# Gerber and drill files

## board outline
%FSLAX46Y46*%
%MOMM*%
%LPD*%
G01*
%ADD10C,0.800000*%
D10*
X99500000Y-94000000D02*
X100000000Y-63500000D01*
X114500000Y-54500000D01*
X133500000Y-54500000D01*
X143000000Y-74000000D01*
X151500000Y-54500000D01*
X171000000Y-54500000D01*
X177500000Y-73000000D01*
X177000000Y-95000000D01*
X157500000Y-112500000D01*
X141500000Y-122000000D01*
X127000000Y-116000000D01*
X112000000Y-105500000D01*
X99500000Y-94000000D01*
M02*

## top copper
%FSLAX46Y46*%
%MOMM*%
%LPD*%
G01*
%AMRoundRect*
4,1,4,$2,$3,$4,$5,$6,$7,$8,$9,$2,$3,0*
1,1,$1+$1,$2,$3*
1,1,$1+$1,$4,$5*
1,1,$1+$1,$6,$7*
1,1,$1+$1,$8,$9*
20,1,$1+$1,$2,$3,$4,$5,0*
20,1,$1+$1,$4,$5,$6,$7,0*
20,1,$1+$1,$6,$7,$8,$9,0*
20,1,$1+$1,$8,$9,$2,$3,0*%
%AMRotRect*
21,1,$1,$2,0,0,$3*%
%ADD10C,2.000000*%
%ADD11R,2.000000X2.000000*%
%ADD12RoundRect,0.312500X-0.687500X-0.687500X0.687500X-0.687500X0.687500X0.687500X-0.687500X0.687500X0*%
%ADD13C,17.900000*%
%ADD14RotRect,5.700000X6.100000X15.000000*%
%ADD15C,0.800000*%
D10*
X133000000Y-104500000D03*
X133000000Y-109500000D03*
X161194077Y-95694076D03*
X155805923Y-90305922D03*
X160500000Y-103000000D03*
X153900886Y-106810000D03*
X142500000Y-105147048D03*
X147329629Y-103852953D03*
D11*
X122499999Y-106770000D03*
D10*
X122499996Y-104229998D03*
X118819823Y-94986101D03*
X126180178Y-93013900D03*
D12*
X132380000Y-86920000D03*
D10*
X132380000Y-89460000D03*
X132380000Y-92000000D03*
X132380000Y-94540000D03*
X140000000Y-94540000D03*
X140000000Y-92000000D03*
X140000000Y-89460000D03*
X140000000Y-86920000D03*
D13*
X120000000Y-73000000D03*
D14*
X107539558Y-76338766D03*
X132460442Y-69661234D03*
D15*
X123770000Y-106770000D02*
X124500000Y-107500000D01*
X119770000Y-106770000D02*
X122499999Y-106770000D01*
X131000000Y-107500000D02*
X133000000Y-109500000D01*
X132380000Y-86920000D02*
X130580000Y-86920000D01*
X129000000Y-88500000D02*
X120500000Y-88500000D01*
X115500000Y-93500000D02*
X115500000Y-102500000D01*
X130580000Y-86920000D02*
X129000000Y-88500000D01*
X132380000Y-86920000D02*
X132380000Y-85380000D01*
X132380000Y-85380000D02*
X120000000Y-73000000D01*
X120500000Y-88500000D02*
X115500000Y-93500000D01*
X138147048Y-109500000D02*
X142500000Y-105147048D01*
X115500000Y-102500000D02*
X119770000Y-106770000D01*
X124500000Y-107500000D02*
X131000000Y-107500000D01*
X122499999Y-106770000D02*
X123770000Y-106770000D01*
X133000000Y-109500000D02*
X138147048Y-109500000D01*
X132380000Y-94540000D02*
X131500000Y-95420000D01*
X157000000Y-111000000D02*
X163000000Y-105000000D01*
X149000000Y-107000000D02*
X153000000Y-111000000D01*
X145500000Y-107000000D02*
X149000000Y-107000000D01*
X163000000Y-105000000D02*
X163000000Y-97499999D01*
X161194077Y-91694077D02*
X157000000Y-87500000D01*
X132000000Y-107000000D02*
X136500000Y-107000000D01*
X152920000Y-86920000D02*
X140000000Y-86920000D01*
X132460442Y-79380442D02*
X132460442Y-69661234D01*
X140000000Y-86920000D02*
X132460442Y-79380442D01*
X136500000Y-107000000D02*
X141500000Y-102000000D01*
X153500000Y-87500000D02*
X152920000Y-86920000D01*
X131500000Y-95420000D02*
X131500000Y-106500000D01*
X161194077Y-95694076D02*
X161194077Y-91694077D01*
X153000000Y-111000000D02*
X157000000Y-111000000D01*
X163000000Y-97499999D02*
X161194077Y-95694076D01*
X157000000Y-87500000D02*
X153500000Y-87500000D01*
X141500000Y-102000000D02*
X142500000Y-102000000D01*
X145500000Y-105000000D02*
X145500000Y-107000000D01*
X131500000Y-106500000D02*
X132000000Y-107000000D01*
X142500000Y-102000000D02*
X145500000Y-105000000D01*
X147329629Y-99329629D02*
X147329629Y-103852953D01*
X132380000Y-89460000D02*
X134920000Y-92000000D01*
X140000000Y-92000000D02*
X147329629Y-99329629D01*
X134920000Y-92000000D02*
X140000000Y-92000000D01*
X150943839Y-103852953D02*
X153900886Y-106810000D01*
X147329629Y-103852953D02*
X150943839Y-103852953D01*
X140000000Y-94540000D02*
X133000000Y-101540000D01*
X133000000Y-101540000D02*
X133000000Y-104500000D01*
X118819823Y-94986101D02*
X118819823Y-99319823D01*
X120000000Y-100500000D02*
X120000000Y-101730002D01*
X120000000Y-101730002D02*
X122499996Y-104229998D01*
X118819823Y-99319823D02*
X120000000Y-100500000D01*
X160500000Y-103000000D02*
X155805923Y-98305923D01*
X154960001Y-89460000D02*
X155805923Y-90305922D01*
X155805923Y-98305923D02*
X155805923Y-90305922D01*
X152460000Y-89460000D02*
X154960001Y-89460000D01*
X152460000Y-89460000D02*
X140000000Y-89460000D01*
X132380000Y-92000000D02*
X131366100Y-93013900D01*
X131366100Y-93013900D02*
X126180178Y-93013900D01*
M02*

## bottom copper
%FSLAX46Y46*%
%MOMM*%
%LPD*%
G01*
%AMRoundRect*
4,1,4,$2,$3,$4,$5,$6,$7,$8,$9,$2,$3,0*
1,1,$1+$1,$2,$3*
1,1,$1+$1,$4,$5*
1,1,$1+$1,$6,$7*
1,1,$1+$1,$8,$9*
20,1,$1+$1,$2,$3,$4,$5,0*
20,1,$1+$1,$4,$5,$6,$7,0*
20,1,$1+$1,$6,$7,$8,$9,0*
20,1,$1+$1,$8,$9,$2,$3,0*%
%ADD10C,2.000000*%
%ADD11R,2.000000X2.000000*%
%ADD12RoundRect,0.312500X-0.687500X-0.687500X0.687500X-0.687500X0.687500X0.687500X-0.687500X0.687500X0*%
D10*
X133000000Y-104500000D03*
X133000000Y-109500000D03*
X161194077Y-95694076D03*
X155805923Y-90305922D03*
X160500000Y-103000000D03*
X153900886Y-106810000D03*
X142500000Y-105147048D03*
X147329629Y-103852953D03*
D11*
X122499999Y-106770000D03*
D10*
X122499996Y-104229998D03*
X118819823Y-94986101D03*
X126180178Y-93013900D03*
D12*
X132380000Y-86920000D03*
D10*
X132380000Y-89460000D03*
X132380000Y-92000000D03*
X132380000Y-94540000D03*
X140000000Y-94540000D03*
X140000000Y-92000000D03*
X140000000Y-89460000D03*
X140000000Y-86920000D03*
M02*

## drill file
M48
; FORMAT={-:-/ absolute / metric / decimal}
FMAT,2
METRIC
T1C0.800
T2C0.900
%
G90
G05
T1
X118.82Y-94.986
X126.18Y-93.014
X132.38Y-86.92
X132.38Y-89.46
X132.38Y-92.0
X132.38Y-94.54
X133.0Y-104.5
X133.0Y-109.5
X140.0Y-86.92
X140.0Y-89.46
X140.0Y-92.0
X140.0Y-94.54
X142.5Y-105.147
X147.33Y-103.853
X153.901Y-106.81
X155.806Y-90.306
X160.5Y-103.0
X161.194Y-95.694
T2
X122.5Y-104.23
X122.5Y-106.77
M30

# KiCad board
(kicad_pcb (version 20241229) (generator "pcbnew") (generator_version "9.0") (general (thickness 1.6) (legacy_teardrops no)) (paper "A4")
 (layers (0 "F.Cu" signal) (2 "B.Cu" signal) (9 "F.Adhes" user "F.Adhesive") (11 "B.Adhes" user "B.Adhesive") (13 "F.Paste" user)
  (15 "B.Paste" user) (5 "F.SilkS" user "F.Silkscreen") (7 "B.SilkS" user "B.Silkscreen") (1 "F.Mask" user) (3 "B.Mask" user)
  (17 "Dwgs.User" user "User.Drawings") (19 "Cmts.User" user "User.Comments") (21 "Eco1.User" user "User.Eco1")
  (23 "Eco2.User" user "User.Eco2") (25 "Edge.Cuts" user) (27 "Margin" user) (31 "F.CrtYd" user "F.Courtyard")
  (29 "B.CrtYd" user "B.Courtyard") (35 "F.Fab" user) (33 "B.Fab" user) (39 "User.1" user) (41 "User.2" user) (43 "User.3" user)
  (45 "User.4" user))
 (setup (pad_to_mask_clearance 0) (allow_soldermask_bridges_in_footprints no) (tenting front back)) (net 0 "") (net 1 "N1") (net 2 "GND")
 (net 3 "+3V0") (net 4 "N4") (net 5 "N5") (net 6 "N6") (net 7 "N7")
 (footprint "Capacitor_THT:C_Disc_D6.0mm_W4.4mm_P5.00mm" (layer "F.Cu") (at 133 104.5 -90)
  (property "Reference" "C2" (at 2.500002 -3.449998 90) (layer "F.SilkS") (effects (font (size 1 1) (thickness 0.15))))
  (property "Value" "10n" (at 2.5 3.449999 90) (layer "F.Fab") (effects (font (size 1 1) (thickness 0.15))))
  (pad "1" thru_hole circle (at 0 0 270) (size 2 2) (drill 0.8) (layers "*.Cu" "*.Mask") (remove_unused_layers no) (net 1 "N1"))
  (pad "2" thru_hole circle (at 5 0 270) (size 2 2) (drill 0.8) (layers "*.Cu" "*.Mask") (remove_unused_layers no) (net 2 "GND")))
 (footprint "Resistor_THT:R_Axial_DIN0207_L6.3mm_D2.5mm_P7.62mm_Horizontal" (layer "F.Cu") (at 161.194077 95.694076 135)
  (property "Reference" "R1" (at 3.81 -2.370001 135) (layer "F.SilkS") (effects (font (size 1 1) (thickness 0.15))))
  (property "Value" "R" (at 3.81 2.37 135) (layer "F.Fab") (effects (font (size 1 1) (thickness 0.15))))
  (pad "1" thru_hole circle (at 0 0 135) (size 2 2) (drill 0.8) (layers "*.Cu" "*.Mask") (remove_unused_layers no) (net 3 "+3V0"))
  (pad "2" thru_hole circle (at 7.62 0 135) (size 2 2) (drill 0.8) (layers "*.Cu" "*.Mask") (remove_unused_layers no) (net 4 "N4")))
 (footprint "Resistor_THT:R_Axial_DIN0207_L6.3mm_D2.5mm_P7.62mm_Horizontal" (layer "F.Cu") (at 160.5 103 -150)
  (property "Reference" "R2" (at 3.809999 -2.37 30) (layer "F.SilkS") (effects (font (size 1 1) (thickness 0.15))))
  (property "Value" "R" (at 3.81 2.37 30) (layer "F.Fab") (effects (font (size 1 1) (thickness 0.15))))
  (pad "1" thru_hole circle (at 0 0 210) (size 2 2) (drill 0.8) (layers "*.Cu" "*.Mask") (remove_unused_layers no) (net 4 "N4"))
  (pad "2" thru_hole circle (at 7.62 0 210) (size 2 2) (drill 0.8) (layers "*.Cu" "*.Mask") (remove_unused_layers no) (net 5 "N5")))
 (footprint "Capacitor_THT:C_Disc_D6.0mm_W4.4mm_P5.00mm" (layer "F.Cu") (at 142.5 105.147048 15)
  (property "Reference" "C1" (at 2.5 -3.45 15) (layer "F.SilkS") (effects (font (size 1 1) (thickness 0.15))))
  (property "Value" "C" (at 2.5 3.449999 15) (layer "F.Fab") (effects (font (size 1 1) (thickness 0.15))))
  (pad "1" thru_hole circle (at 0 0 15) (size 2 2) (drill 0.8) (layers "*.Cu" "*.Mask") (remove_unused_layers no) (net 2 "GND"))
  (pad "2" thru_hole circle (at 5 0 15) (size 2 2) (drill 0.8) (layers "*.Cu" "*.Mask") (remove_unused_layers no) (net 5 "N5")))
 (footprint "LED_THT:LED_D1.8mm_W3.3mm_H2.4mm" (layer "F.Cu") (at 122.499999 106.77 90)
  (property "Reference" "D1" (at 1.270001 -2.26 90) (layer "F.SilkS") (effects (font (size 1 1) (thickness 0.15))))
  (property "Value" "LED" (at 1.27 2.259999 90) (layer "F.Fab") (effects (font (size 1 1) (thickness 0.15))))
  (pad "1" thru_hole rect (at 0 0 90) (size 2 2) (drill 0.9) (layers "*.Cu" "*.Mask") (remove_unused_layers no) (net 2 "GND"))
  (pad "2" thru_hole circle (at 2.540002 -0.000003 90) (size 2 2) (drill 0.9) (layers "*.Cu" "*.Mask") (remove_unused_layers no)
   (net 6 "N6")))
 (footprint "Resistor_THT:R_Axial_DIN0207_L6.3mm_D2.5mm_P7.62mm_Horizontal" (layer "F.Cu") (at 118.819823 94.986101 15)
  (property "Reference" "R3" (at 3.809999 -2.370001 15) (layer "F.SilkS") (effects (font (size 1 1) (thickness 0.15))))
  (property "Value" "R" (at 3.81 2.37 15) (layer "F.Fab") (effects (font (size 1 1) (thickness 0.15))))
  (pad "1" thru_hole circle (at 0 0 15) (size 2 2) (drill 0.8) (layers "*.Cu" "*.Mask") (remove_unused_layers no) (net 6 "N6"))
  (pad "2" thru_hole circle (at 7.62 0 15) (size 2 2) (drill 0.8) (layers "*.Cu" "*.Mask") (remove_unused_layers no) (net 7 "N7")))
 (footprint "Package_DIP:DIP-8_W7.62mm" (layer "F.Cu") (at 132.38 86.92)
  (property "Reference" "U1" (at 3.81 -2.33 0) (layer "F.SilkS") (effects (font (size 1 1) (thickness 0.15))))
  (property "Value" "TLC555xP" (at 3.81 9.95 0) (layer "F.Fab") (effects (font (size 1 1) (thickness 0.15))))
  (pad "1" thru_hole roundrect (at 0 0) (size 2 2) (drill 0.8) (layers "*.Cu" "*.Mask") (remove_unused_layers no) (roundrect_rratio 0.15625)
   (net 2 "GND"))
  (pad "2" thru_hole circle (at 0 2.54) (size 2 2) (drill 0.8) (layers "*.Cu" "*.Mask") (remove_unused_layers no) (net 5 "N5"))
  (pad "3" thru_hole circle (at 0 5.08) (size 2 2) (drill 0.8) (layers "*.Cu" "*.Mask") (remove_unused_layers no) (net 7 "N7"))
  (pad "4" thru_hole circle (at 0 7.62) (size 2 2) (drill 0.8) (layers "*.Cu" "*.Mask") (remove_unused_layers no) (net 3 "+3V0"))
  (pad "5" thru_hole circle (at 7.62 7.62) (size 2 2) (drill 0.8) (layers "*.Cu" "*.Mask") (remove_unused_layers no) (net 1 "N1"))
  (pad "6" thru_hole circle (at 7.62 5.08) (size 2 2) (drill 0.8) (layers "*.Cu" "*.Mask") (remove_unused_layers no) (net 5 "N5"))
  (pad "7" thru_hole circle (at 7.62 2.54) (size 2 2) (drill 0.8) (layers "*.Cu" "*.Mask") (remove_unused_layers no) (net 4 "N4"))
  (pad "8" thru_hole circle (at 7.62 0) (size 2 2) (drill 0.8) (layers "*.Cu" "*.Mask") (remove_unused_layers no) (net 3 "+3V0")))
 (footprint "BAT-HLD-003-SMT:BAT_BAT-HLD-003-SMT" (layer "F.Cu") (at 120 73 15)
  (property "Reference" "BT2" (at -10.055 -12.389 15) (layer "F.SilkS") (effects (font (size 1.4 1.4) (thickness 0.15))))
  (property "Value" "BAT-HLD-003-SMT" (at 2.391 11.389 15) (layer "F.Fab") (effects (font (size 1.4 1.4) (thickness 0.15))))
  (pad "N" smd circle (at 0 0 15) (size 17.9 17.9) (layers "F.Cu" "F.Mask") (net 2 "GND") (solder_mask_margin 0.102))
  (pad "P1" smd rect (at -12.899999 0.000001 15) (size 5.7 6.1) (layers "F.Cu" "F.Mask" "F.Paste") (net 3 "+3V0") (solder_mask_margin 0.102))
  (pad "P2" smd rect (at 12.899999 -0.000001 15) (size 5.7 6.1) (layers "F.Cu" "F.Mask" "F.Paste") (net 3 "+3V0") (solder_mask_margin 0.102)))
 (gr_poly
  (pts (xy 99.5 94) (xy 100 63.5) (xy 114.5 54.5) (xy 133.5 54.5) (xy 143 74) (xy 151.5 54.5) (xy 171 54.5) (xy 177.5 73) (xy 177 95)
   (xy 157.5 112.5) (xy 141.5 122) (xy 127 116) (xy 112 105.5))
  (stroke (width 0.8) (type solid)) (fill no) (layer "Edge.Cuts"))
 (segment (start 123.77 106.77) (end 124.5 107.5) (width 0.8) (layer "F.Cu") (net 2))
 (segment (start 119.77 106.77) (end 122.499999 106.77) (width 0.8) (layer "F.Cu") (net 2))
 (segment (start 131 107.5) (end 133 109.5) (width 0.8) (layer "F.Cu") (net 2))
 (segment (start 132.38 86.92) (end 130.58 86.92) (width 0.8) (layer "F.Cu") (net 2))
 (segment (start 129 88.5) (end 120.5 88.5) (width 0.8) (layer "F.Cu") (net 2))
 (segment (start 115.5 93.5) (end 115.5 102.5) (width 0.8) (layer "F.Cu") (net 2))
 (segment (start 130.58 86.92) (end 129 88.5) (width 0.8) (layer "F.Cu") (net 2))
 (segment (start 132.38 86.92) (end 132.38 85.38) (width 0.8) (layer "F.Cu") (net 2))
 (segment (start 132.38 85.38) (end 120 73) (width 0.8) (layer "F.Cu") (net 2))
 (segment (start 120.5 88.5) (end 115.5 93.5) (width 0.8) (layer "F.Cu") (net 2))
 (segment (start 138.147048 109.5) (end 142.5 105.147048) (width 0.8) (layer "F.Cu") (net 2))
 (segment (start 115.5 102.5) (end 119.77 106.77) (width 0.8) (layer "F.Cu") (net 2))
 (segment (start 124.5 107.5) (end 131 107.5) (width 0.8) (layer "F.Cu") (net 2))
 (segment (start 122.499999 106.77) (end 123.77 106.77) (width 0.8) (layer "F.Cu") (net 2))
 (segment (start 133 109.5) (end 138.147048 109.5) (width 0.8) (layer "F.Cu") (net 2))
 (segment (start 132.38 94.54) (end 131.5 95.42) (width 0.8) (layer "F.Cu") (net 3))
 (segment (start 157 111) (end 163 105) (width 0.8) (layer "F.Cu") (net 3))
 (segment (start 149 107) (end 153 111) (width 0.8) (layer "F.Cu") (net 3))
 (segment (start 145.5 107) (end 149 107) (width 0.8) (layer "F.Cu") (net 3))
 (segment (start 163 105) (end 163 97.499999) (width 0.8) (layer "F.Cu") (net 3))
 (segment (start 161.194077 91.694077) (end 157 87.5) (width 0.8) (layer "F.Cu") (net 3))
 (segment (start 132 107) (end 136.5 107) (width 0.8) (layer "F.Cu") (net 3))
 (segment (start 152.92 86.92) (end 140 86.92) (width 0.8) (layer "F.Cu") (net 3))
 (segment (start 132.460442 79.380442) (end 132.460442 69.661234) (width 0.8) (layer "F.Cu") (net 3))
 (segment (start 140 86.92) (end 132.460442 79.380442) (width 0.8) (layer "F.Cu") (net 3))
 (segment (start 136.5 107) (end 141.5 102) (width 0.8) (layer "F.Cu") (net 3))
 (segment (start 153.5 87.5) (end 152.92 86.92) (width 0.8) (layer "F.Cu") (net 3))
 (segment (start 131.5 95.42) (end 131.5 106.5) (width 0.8) (layer "F.Cu") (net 3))
 (segment (start 161.194077 95.694076) (end 161.194077 91.694077) (width 0.8) (layer "F.Cu") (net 3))
 (segment (start 153 111) (end 157 111) (width 0.8) (layer "F.Cu") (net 3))
 (segment (start 163 97.499999) (end 161.194077 95.694076) (width 0.8) (layer "F.Cu") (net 3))
 (segment (start 157 87.5) (end 153.5 87.5) (width 0.8) (layer "F.Cu") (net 3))
 (segment (start 141.5 102) (end 142.5 102) (width 0.8) (layer "F.Cu") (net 3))
 (segment (start 145.5 105) (end 145.5 107) (width 0.8) (layer "F.Cu") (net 3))
 (segment (start 131.5 106.5) (end 132 107) (width 0.8) (layer "F.Cu") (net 3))
 (segment (start 142.5 102) (end 145.5 105) (width 0.8) (layer "F.Cu") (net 3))
 (segment (start 147.329629 99.329629) (end 147.329629 103.852953) (width 0.8) (layer "F.Cu") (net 5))
 (segment (start 132.38 89.46) (end 134.92 92) (width 0.8) (layer "F.Cu") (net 5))
 (segment (start 140 92) (end 147.329629 99.329629) (width 0.8) (layer "F.Cu") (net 5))
 (segment (start 134.92 92) (end 140 92) (width 0.8) (layer "F.Cu") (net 5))
 (segment (start 150.943839 103.852953) (end 153.900886 106.81) (width 0.8) (layer "F.Cu") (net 5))
 (segment (start 147.329629 103.852953) (end 150.943839 103.852953) (width 0.8) (layer "F.Cu") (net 5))
 (segment (start 140 94.54) (end 133 101.54) (width 0.8) (layer "F.Cu") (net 1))
 (segment (start 133 101.54) (end 133 104.5) (width 0.8) (layer "F.Cu") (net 1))
 (segment (start 118.819823 94.986101) (end 118.819823 99.319823) (width 0.8) (layer "F.Cu") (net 6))
 (segment (start 120 100.5) (end 120 101.730002) (width 0.8) (layer "F.Cu") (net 6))
 (segment (start 120 101.730002) (end 122.499996 104.229998) (width 0.8) (layer "F.Cu") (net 6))
 (segment (start 118.819823 99.319823) (end 120 100.5) (width 0.8) (layer "F.Cu") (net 6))
 (segment (start 160.5 103) (end 155.805923 98.305923) (width 0.8) (layer "F.Cu") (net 4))
 (segment (start 154.960001 89.46) (end 155.805923 90.305922) (width 0.8) (layer "F.Cu") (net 4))
 (segment (start 155.805923 98.305923) (end 155.805923 90.305922) (width 0.8) (layer "F.Cu") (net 4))
 (segment (start 152.46 89.46) (end 154.960001 89.46) (width 0.8) (layer "F.Cu") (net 4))
 (segment (start 152.46 89.46) (end 140 89.46) (width 0.8) (layer "F.Cu") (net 4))
 (segment (start 132.38 92) (end 131.3661 93.0139) (width 0.8) (layer "F.Cu") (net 7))
 (segment (start 131.3661 93.0139) (end 126.180178 93.0139) (width 0.8) (layer "F.Cu") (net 7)))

